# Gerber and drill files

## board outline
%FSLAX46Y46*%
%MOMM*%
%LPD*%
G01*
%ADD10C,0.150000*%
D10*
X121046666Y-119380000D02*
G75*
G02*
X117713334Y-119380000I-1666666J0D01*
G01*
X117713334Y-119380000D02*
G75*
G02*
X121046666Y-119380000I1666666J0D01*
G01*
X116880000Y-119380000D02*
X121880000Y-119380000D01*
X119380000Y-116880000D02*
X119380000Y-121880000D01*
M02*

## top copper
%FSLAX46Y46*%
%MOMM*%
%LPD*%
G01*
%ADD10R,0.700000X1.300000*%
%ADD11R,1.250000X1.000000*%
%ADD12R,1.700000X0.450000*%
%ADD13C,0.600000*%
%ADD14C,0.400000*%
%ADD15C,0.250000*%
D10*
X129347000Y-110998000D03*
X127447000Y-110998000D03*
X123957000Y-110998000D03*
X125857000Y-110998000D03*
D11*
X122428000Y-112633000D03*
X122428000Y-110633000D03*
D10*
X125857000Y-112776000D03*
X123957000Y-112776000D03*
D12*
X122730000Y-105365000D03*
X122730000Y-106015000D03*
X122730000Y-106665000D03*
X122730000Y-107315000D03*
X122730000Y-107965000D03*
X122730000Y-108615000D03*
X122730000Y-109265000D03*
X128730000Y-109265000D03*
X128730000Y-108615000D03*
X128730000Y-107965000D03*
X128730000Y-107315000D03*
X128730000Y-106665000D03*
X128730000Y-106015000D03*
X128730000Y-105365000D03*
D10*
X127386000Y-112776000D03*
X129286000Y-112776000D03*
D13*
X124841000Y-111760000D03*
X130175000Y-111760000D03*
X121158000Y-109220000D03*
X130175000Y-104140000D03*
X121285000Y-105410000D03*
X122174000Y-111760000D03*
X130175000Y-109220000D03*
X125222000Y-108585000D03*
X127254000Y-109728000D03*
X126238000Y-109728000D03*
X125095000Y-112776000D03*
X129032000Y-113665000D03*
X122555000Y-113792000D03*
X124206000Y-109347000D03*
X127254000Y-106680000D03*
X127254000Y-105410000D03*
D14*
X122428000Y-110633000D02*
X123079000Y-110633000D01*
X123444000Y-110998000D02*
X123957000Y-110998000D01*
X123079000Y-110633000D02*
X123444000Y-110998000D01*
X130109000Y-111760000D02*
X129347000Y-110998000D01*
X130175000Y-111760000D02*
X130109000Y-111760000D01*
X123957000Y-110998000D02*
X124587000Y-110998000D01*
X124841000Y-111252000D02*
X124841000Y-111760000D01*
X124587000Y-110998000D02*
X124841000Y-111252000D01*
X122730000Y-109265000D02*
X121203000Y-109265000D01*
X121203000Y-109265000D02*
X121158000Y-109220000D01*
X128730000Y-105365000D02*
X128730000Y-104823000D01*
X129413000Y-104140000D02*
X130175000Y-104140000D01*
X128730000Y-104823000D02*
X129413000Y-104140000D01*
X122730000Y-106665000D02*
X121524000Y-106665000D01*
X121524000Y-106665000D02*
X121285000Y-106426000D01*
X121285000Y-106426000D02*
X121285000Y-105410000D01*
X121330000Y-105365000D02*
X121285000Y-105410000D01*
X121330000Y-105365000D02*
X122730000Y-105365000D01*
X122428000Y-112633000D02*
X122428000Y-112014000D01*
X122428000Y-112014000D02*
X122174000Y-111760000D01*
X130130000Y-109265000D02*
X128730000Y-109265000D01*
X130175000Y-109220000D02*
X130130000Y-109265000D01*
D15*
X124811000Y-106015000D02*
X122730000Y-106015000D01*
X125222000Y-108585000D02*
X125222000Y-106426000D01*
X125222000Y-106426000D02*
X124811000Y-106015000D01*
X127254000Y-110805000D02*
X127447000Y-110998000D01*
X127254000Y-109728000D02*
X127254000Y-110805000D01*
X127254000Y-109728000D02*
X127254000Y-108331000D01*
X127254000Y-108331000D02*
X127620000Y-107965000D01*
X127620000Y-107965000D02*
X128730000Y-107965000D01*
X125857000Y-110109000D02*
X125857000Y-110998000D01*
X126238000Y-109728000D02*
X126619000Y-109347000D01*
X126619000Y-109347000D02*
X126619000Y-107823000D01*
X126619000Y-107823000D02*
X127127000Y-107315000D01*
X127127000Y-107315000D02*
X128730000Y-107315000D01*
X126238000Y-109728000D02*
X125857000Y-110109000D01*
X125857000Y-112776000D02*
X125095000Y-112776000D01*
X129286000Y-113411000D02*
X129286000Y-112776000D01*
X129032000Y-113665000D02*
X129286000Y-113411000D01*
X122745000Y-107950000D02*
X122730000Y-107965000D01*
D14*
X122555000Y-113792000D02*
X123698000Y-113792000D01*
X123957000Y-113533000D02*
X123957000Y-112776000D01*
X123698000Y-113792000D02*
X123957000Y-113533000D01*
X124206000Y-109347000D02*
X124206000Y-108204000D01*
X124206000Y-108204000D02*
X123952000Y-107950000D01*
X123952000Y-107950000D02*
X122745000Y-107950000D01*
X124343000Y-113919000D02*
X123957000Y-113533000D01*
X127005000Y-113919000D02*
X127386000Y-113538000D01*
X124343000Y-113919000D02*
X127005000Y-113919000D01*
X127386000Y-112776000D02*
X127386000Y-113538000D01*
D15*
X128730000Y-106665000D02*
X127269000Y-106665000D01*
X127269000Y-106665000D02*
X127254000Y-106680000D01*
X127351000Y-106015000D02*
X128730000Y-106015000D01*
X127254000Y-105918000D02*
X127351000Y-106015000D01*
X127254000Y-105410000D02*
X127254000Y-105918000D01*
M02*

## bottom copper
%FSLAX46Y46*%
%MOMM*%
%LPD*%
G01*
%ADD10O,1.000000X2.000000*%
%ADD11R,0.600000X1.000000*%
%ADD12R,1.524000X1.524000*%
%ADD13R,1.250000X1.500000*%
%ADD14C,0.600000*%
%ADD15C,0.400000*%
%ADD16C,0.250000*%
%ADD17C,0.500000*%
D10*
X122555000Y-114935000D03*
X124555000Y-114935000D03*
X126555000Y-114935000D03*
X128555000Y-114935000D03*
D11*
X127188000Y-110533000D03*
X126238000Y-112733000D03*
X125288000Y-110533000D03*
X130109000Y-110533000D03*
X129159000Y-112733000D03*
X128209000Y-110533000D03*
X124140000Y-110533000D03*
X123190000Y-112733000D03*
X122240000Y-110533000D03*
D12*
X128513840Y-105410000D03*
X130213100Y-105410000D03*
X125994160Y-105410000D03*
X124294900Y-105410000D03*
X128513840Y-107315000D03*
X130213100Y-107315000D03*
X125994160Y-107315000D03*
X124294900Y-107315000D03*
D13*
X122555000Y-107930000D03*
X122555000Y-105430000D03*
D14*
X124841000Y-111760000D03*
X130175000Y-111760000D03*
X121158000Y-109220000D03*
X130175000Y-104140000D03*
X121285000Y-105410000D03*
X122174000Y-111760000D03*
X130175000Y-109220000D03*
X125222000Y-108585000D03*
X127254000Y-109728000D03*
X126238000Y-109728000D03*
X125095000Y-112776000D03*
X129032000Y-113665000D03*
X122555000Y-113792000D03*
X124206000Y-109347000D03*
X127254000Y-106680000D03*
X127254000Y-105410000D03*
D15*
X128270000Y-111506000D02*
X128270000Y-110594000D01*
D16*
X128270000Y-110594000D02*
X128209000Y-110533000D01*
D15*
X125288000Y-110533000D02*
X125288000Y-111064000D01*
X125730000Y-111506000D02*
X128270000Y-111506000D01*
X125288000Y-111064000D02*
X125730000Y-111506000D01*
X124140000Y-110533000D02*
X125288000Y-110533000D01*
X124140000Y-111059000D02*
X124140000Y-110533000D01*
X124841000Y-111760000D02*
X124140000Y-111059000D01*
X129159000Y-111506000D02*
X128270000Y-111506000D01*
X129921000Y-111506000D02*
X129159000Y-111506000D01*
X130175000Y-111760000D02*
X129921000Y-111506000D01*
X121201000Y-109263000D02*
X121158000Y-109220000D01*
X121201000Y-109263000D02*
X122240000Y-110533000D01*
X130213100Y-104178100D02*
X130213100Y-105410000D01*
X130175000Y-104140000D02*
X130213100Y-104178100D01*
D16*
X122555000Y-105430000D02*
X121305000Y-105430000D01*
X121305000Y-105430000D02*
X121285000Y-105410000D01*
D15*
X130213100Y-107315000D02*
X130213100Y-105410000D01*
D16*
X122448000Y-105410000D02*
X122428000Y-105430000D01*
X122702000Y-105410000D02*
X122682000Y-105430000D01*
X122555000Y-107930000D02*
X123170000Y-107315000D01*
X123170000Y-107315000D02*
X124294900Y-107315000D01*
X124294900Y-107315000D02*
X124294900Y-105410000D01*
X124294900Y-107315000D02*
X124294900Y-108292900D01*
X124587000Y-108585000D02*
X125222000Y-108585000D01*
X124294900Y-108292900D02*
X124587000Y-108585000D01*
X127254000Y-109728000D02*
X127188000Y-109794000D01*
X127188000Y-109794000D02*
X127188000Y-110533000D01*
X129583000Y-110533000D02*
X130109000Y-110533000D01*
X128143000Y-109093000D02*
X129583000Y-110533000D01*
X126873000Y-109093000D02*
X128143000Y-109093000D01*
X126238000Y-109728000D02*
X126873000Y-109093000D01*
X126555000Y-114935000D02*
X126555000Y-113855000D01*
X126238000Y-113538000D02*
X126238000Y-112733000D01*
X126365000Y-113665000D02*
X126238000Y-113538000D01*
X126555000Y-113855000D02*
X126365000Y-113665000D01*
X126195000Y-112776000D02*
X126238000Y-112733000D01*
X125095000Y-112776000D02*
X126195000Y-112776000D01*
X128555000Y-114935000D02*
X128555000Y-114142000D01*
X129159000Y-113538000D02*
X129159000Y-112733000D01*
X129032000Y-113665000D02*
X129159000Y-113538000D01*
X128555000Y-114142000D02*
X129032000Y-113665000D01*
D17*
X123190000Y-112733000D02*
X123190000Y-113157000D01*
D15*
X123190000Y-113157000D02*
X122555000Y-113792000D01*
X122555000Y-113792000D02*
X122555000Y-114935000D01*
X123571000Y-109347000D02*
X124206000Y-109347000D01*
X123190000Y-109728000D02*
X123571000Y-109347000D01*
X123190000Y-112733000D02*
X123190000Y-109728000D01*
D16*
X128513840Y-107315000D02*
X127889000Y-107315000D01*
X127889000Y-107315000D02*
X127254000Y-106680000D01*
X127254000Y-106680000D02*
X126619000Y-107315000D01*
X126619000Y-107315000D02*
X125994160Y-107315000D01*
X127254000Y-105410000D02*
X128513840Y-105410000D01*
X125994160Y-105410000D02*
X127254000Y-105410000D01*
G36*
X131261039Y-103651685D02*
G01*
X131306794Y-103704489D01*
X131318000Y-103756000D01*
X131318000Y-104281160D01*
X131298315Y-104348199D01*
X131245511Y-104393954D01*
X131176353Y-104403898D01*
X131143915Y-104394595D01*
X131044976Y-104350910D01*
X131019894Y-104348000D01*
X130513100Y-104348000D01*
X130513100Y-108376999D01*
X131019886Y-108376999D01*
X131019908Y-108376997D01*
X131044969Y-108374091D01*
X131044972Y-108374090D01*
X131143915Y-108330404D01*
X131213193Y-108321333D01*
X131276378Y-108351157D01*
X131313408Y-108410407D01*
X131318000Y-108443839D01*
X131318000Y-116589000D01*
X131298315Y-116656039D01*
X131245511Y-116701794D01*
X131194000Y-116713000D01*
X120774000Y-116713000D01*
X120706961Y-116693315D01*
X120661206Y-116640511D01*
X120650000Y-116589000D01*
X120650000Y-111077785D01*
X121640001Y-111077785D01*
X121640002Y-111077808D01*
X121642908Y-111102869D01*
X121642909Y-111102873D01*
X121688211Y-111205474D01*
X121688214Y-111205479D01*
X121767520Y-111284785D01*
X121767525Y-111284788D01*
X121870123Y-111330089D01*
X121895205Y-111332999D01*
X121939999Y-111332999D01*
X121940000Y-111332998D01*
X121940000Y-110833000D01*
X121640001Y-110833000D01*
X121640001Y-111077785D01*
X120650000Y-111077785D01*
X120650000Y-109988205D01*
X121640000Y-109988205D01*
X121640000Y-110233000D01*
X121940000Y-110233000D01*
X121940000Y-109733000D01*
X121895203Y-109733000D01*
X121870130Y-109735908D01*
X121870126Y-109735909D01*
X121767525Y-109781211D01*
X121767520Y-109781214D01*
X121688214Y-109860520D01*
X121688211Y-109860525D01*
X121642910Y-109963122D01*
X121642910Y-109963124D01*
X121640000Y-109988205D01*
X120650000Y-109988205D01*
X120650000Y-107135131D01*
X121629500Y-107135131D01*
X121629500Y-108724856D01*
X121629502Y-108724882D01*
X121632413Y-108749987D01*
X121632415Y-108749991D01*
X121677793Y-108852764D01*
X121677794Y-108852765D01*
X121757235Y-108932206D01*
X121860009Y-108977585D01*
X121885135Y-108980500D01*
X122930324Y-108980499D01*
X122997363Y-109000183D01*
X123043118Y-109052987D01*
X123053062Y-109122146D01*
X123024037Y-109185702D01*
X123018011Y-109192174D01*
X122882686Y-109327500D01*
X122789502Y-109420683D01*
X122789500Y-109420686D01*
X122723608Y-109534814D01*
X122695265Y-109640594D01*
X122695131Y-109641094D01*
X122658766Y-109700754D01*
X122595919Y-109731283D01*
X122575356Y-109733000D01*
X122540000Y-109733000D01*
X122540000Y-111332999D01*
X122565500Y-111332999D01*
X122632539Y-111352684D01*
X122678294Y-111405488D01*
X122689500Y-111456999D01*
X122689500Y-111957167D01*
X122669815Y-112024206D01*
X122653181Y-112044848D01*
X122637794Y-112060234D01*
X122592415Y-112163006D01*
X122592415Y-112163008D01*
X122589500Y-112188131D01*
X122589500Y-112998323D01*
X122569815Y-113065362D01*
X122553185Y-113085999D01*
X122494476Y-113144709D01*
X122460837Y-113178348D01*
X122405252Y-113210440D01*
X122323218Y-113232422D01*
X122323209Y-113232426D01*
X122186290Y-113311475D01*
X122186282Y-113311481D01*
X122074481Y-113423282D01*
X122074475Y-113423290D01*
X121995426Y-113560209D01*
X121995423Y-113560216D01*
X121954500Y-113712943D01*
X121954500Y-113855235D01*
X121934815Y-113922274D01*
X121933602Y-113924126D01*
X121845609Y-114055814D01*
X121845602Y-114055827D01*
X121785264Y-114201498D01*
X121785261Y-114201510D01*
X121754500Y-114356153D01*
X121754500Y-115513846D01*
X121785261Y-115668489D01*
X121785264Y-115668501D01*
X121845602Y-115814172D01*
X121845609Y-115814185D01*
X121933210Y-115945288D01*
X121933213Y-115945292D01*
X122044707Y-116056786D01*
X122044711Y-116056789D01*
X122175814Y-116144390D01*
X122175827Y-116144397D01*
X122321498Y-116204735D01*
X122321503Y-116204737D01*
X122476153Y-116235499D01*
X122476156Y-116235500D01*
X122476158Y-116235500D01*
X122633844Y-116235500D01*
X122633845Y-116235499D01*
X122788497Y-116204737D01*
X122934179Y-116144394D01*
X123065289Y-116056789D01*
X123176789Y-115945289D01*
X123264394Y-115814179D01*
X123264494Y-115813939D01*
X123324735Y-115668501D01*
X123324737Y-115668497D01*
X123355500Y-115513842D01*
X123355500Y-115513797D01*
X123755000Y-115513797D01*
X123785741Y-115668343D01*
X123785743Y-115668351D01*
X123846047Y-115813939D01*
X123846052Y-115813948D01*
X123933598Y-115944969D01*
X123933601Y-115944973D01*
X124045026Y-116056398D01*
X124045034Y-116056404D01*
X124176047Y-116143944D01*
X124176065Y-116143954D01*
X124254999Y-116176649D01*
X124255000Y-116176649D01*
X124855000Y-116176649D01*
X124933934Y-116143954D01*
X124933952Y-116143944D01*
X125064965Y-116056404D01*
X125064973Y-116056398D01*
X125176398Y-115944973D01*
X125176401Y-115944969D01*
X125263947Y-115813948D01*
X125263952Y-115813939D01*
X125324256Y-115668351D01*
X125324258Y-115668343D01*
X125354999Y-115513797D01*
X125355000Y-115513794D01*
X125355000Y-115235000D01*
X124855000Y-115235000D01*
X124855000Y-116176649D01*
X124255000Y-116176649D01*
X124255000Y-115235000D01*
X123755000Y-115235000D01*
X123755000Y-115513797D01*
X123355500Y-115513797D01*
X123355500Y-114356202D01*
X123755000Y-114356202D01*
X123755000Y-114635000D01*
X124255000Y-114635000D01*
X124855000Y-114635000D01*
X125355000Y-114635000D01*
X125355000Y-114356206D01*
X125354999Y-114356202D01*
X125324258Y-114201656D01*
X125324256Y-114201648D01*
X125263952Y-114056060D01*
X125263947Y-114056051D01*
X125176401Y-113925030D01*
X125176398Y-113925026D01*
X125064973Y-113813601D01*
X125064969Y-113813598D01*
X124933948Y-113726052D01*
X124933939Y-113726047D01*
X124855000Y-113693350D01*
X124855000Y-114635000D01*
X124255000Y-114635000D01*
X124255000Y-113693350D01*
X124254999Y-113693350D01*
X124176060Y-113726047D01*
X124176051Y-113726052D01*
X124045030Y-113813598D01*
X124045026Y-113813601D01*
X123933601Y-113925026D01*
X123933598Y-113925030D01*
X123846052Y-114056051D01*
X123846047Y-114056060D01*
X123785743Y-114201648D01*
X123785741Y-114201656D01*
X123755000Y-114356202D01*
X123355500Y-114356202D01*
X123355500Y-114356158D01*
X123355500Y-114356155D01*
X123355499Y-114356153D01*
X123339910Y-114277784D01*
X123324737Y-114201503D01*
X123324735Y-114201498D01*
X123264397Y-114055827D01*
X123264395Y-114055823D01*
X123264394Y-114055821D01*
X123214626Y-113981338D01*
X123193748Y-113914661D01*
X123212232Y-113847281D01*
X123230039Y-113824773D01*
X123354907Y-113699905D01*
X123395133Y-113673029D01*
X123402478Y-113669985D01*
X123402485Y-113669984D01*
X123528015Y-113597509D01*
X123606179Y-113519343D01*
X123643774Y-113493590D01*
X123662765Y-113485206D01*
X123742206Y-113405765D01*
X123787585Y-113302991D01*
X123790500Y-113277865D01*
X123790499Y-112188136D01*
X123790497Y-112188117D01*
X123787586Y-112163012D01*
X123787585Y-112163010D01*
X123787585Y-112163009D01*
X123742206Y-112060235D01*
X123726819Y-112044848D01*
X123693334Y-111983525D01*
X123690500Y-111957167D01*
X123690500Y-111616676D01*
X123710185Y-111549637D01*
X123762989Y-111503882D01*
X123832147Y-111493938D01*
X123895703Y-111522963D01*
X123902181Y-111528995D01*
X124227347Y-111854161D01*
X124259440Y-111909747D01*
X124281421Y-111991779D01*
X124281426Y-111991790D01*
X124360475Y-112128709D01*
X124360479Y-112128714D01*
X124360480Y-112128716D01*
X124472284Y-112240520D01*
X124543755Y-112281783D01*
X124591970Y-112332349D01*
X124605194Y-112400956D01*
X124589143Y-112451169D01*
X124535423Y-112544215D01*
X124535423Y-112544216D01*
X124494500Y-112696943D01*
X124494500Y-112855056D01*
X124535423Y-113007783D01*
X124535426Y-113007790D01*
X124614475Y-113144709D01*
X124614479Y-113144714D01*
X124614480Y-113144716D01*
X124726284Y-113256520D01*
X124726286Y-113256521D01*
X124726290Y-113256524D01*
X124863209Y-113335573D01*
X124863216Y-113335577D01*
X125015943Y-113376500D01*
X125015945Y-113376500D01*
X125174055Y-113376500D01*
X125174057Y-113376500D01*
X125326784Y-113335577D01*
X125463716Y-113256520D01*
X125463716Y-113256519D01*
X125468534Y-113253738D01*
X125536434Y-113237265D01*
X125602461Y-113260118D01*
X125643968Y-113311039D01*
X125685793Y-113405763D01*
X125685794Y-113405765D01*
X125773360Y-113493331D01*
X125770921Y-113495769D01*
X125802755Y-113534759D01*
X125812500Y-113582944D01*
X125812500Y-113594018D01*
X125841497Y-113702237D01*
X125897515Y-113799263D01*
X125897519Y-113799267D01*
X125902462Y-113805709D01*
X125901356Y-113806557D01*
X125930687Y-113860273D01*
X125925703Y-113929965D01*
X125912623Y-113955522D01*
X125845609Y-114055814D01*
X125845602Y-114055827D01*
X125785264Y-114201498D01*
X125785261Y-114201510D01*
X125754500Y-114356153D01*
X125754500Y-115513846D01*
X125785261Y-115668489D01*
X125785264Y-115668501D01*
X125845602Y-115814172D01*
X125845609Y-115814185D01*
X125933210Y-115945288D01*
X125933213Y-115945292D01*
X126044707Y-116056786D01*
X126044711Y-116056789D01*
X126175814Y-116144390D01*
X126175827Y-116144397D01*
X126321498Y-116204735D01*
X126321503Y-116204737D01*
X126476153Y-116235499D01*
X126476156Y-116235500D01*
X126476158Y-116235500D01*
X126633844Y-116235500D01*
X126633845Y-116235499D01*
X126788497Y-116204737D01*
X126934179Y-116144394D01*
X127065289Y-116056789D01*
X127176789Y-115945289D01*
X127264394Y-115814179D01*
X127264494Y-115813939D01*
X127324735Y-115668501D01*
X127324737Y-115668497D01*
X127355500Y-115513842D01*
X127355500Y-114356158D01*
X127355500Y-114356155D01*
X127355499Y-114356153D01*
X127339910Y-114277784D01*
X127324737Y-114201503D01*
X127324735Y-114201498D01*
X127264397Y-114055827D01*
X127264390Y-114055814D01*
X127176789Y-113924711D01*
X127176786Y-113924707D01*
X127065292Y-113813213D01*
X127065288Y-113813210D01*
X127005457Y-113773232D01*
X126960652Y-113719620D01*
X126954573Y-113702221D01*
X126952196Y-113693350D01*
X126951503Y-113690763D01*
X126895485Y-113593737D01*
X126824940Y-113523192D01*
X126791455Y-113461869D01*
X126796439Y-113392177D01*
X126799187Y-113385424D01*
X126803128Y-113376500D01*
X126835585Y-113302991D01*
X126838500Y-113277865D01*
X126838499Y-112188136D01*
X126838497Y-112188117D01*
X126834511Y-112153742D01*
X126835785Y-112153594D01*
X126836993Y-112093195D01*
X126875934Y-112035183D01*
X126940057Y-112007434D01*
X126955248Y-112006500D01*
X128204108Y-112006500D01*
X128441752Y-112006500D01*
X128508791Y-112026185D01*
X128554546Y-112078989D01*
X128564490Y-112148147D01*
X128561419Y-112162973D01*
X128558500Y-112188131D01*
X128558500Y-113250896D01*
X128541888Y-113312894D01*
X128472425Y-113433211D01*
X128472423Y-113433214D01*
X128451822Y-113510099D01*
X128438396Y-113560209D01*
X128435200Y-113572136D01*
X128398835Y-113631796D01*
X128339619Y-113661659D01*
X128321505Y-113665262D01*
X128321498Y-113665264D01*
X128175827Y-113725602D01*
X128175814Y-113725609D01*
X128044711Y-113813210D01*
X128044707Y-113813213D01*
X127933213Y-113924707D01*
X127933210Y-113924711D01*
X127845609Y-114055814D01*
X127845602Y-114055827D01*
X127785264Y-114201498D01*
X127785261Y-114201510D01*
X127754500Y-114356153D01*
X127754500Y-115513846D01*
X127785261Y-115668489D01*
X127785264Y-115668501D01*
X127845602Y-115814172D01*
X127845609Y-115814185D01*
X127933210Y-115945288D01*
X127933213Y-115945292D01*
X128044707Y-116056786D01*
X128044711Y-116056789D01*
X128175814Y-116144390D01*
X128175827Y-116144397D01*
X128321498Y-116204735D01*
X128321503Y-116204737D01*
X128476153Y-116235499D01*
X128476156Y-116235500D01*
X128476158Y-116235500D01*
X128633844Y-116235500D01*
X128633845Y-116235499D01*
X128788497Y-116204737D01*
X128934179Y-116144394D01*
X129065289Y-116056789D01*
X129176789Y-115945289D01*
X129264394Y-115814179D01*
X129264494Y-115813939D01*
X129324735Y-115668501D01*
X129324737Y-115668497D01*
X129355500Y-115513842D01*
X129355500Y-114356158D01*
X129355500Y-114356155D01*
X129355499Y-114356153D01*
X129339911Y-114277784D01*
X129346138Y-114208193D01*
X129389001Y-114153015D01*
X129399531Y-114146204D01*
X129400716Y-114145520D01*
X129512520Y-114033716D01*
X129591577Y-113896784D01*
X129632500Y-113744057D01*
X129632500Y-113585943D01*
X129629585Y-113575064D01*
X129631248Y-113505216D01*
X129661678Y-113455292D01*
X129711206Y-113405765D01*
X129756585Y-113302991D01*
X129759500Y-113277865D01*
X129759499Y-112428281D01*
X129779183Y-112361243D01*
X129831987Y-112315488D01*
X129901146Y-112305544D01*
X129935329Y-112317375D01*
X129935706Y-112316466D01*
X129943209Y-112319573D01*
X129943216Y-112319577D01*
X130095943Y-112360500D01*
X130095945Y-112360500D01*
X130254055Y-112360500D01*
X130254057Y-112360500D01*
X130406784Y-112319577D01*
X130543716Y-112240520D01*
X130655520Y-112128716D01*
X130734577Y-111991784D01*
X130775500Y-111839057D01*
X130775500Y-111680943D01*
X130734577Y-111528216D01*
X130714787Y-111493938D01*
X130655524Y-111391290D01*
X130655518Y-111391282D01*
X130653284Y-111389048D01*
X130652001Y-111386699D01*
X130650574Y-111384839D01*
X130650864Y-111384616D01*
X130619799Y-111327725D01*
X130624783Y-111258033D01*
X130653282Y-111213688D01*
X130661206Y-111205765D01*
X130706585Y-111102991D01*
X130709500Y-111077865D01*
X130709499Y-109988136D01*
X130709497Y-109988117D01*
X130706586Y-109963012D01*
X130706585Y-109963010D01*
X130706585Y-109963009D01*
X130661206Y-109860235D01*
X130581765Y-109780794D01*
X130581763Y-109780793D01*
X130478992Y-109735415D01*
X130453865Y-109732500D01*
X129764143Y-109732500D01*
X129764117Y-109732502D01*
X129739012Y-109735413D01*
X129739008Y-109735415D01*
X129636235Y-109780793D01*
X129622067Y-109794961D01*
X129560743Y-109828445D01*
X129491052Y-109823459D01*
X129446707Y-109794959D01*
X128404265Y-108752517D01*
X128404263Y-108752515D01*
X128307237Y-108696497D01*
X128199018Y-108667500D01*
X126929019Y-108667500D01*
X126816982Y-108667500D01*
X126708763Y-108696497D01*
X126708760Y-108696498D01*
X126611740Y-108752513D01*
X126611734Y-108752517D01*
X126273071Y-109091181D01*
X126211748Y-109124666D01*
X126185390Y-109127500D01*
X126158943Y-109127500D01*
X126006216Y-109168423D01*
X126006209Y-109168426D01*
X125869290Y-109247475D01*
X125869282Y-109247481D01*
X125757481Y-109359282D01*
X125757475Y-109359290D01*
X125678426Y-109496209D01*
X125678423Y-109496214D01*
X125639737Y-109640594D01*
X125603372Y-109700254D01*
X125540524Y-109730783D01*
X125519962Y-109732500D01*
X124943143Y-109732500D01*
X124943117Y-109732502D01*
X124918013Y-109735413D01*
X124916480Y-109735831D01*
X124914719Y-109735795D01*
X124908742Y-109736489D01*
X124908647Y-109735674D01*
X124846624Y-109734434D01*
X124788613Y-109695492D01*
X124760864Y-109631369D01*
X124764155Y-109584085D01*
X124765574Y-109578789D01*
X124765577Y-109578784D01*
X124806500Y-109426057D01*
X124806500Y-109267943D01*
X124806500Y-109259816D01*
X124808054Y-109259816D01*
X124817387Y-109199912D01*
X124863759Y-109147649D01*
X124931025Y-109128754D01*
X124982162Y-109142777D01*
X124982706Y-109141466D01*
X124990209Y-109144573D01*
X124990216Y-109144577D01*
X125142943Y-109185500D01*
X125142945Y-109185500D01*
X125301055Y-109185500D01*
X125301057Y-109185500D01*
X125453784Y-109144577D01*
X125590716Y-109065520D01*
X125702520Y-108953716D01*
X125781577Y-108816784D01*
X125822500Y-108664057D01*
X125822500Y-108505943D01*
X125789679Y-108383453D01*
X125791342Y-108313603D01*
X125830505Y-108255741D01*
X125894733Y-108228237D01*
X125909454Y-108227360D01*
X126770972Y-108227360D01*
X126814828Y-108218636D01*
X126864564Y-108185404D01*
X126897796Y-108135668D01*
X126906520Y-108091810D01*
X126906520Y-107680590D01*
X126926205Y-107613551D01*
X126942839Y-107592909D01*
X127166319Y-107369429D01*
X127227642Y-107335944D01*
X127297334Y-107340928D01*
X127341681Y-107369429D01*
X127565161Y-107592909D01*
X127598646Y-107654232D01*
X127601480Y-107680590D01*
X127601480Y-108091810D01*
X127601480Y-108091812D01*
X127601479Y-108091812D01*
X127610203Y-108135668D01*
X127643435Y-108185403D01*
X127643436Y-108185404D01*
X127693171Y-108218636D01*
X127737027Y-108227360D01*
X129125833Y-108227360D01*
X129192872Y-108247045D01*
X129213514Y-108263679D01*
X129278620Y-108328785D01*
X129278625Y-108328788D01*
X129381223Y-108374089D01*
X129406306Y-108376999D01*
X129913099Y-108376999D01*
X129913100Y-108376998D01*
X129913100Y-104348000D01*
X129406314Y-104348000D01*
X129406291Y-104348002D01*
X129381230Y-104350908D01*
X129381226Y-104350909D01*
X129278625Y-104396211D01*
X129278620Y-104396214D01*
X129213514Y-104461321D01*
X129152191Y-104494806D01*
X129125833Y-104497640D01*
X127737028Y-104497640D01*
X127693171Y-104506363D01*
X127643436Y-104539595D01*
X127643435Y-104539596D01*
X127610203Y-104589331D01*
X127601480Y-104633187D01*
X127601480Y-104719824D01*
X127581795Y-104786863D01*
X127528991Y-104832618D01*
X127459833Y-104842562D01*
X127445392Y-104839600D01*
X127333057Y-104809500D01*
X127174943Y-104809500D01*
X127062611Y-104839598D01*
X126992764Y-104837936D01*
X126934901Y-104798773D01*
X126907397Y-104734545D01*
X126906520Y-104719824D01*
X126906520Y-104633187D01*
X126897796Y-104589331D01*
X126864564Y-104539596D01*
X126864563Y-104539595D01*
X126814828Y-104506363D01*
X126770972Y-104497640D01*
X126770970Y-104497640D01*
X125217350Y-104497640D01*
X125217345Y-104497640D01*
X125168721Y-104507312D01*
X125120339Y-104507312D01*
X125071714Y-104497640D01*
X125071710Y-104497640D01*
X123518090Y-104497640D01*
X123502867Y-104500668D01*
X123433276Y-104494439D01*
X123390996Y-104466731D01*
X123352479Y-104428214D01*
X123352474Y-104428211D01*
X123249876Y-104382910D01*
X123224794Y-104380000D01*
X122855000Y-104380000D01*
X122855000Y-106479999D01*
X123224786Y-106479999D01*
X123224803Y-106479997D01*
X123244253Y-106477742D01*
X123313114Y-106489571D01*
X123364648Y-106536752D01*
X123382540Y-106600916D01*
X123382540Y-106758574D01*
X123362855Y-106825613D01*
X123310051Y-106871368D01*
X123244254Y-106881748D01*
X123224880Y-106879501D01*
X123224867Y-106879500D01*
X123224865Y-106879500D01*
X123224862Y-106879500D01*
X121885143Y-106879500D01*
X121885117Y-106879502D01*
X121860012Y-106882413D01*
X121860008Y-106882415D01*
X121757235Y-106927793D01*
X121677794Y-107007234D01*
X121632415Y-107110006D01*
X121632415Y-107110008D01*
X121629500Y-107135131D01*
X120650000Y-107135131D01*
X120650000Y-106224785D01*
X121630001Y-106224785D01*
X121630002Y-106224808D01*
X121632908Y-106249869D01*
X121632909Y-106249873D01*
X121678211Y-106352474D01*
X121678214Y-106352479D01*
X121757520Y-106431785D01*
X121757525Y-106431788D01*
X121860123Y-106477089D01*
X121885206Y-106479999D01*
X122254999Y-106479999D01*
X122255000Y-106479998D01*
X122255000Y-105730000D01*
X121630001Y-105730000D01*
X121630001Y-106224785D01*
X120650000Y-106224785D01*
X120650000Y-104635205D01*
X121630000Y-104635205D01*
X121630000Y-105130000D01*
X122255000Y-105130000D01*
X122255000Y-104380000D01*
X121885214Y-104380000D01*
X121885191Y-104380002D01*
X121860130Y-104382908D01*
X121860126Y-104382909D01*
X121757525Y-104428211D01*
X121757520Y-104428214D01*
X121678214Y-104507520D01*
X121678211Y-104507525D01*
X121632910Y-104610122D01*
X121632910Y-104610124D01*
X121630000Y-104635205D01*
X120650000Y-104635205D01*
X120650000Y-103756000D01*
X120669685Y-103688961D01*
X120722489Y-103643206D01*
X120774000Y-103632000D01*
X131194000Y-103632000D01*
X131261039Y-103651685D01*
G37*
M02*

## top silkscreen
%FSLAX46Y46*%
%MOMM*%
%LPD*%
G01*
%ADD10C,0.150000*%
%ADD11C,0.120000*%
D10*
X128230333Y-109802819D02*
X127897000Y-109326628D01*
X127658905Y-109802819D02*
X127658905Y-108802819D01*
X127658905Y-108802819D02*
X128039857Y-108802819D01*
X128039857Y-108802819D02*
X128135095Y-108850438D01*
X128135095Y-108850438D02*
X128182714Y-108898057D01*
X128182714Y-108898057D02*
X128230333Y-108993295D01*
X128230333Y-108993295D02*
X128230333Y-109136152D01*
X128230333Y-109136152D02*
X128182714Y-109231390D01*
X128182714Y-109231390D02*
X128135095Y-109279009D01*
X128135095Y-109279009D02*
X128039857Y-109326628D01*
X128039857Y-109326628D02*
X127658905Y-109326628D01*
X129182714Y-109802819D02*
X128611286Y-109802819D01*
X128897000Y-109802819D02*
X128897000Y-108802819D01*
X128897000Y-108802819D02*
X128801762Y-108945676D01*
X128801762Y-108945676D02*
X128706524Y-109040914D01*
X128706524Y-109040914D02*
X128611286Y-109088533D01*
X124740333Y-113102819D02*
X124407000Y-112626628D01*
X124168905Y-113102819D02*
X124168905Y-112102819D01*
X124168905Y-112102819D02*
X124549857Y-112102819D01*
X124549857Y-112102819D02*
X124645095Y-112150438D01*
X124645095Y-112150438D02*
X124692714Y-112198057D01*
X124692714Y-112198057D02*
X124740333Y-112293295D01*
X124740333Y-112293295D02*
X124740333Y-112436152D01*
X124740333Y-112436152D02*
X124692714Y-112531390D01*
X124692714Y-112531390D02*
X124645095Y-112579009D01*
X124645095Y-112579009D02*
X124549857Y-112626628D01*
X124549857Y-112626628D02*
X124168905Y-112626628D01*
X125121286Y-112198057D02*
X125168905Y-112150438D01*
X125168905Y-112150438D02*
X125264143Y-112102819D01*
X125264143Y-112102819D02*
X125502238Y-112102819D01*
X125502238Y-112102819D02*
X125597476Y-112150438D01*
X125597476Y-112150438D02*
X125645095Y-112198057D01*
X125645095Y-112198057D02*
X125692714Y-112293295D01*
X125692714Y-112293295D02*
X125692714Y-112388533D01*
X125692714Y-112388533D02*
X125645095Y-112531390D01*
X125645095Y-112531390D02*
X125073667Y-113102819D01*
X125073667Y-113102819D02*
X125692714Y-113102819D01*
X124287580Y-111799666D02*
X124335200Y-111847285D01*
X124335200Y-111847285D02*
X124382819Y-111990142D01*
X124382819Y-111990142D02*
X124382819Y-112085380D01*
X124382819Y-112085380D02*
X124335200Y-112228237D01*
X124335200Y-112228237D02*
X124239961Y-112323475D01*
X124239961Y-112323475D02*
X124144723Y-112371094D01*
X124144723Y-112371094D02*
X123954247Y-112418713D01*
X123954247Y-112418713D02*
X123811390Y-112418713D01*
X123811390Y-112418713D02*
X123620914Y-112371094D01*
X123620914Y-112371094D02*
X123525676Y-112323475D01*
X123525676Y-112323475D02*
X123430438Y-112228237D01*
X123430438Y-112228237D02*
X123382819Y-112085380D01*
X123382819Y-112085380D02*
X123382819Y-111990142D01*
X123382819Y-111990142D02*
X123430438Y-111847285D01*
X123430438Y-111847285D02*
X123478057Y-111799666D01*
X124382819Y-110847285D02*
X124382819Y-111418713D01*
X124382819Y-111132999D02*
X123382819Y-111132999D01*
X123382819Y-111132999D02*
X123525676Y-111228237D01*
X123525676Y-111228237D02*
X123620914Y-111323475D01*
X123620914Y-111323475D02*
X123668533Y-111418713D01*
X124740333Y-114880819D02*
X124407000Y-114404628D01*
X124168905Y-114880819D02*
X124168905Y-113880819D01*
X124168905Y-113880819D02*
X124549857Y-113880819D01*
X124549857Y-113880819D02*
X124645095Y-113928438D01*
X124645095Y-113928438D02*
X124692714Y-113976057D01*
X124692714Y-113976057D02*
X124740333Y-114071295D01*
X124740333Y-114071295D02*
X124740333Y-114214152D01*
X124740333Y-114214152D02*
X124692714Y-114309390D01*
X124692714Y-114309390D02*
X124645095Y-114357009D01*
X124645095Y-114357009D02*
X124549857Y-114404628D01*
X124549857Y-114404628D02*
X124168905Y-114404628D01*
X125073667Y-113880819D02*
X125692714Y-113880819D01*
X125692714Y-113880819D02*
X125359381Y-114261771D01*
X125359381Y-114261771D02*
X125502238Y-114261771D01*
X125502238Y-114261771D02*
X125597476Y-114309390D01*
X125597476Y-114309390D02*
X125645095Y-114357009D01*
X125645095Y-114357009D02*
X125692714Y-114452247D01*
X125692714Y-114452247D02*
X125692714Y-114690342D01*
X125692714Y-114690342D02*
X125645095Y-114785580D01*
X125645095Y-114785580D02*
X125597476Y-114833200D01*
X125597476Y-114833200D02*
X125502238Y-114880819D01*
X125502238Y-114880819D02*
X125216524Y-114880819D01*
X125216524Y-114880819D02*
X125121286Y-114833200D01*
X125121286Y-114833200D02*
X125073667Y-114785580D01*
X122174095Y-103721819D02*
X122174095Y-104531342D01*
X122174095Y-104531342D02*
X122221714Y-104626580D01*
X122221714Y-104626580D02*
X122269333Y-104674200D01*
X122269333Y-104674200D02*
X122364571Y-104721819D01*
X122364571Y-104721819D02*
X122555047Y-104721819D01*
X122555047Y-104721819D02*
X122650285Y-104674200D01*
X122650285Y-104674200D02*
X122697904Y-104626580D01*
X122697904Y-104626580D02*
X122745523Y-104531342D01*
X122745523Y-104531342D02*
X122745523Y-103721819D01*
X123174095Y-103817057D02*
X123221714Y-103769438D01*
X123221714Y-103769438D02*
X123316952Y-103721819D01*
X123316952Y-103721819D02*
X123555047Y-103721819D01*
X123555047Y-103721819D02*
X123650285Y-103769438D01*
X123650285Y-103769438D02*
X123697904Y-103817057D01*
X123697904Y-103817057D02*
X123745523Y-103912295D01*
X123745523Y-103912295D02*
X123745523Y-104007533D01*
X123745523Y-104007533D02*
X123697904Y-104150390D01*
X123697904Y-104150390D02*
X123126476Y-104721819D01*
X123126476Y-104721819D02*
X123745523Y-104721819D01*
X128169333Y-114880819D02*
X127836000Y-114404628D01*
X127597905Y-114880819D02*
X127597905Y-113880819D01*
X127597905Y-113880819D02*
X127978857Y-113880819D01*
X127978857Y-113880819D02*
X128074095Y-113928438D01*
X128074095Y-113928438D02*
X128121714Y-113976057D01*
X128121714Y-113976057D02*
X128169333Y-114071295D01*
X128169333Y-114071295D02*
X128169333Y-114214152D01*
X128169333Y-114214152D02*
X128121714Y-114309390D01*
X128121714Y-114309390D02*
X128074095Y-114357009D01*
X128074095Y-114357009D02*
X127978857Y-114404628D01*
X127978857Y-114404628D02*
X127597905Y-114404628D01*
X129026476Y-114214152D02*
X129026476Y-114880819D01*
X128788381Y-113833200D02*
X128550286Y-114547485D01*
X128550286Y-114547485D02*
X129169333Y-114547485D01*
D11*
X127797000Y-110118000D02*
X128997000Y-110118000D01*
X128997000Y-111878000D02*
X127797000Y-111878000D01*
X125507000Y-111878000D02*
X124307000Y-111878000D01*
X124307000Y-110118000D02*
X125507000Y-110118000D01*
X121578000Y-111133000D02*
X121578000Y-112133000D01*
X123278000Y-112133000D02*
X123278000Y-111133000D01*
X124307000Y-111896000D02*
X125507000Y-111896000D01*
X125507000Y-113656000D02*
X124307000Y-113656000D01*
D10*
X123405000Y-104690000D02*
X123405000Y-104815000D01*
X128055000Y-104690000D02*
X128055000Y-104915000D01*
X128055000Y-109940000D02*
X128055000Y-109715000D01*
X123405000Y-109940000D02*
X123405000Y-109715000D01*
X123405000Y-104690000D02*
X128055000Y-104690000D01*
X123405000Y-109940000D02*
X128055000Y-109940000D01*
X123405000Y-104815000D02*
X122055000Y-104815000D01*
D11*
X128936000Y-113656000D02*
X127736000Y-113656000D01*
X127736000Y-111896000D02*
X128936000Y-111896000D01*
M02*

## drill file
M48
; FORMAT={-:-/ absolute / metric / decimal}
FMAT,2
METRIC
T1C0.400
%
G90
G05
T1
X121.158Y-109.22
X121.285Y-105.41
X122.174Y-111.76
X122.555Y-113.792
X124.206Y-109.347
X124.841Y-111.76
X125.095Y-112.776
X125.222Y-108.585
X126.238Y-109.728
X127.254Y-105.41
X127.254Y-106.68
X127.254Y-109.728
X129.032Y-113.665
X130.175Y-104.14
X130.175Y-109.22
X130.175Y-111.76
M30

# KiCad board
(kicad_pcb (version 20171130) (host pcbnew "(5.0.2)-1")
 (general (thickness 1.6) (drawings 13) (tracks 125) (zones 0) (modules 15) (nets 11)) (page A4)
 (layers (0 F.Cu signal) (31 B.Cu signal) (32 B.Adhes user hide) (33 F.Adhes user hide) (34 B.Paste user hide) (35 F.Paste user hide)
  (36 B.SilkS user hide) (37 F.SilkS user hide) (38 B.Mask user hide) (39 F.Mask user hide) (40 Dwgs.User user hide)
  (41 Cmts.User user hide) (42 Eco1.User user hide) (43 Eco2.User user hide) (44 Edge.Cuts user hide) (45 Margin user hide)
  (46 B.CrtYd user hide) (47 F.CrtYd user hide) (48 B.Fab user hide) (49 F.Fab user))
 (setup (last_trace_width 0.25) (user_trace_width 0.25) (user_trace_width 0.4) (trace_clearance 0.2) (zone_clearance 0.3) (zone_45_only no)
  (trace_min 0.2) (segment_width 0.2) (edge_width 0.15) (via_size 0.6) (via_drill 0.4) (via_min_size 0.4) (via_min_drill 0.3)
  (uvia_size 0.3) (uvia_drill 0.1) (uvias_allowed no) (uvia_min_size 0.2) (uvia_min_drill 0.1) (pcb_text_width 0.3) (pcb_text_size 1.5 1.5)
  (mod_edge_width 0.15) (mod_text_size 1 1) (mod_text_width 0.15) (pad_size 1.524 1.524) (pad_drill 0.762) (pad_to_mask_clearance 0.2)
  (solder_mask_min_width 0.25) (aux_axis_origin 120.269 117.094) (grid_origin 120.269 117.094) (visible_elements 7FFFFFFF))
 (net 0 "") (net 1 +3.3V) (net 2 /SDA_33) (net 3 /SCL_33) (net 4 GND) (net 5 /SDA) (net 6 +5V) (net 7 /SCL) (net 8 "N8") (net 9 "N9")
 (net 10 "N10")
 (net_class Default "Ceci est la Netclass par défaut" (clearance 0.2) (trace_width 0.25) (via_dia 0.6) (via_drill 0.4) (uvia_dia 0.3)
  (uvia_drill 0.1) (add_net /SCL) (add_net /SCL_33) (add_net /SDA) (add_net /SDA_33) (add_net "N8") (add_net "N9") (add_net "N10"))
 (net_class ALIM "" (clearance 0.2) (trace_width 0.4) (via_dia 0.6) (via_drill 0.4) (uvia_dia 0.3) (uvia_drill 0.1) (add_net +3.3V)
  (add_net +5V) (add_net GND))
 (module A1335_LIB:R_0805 (layer F.Cu) (at 128.397 110.998)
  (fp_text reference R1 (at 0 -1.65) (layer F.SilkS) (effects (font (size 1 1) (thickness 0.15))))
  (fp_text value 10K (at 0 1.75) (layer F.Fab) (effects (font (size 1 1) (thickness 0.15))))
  (fp_line (start -0.6 -0.88) (end 0.6 -0.88) (layer F.SilkS) (width 0.12))
  (fp_line (start 0.6 0.88) (end -0.6 0.88) (layer F.SilkS) (width 0.12))
  (pad 2 smd rect (at 0.95 0) (size 0.7 1.3) (layers F.Cu F.Paste F.Mask) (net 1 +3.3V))
  (pad 1 smd rect (at -0.95 0) (size 0.7 1.3) (layers F.Cu F.Paste F.Mask) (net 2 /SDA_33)))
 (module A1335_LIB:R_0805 (layer F.Cu) (at 124.907 110.998 180)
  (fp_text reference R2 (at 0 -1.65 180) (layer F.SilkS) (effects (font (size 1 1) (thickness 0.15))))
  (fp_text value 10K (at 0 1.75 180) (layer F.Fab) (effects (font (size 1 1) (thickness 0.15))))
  (fp_line (start -0.6 -0.88) (end 0.6 -0.88) (layer F.SilkS) (width 0.12))
  (fp_line (start 0.6 0.88) (end -0.6 0.88) (layer F.SilkS) (width 0.12))
  (pad 2 smd rect (at 0.95 0 180) (size 0.7 1.3) (layers F.Cu F.Paste F.Mask) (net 1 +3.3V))
  (pad 1 smd rect (at -0.95 0 180) (size 0.7 1.3) (layers F.Cu F.Paste F.Mask) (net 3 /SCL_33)))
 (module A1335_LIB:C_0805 (layer F.Cu) (at 122.428 111.633 270)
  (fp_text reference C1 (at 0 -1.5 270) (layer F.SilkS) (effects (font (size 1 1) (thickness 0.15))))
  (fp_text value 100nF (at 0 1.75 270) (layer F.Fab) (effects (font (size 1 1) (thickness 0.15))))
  (fp_line (start -0.5 0.85) (end 0.5 0.85) (layer F.SilkS) (width 0.12))
  (fp_line (start 0.5 -0.85) (end -0.5 -0.85) (layer F.SilkS) (width 0.12))
  (pad 2 smd rect (at 1 0 270) (size 1 1.25) (layers F.Cu F.Paste F.Mask) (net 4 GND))
  (pad 1 smd rect (at -1 0 270) (size 1 1.25) (layers F.Cu F.Paste F.Mask) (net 1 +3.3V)))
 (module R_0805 (layer F.Cu) (at 124.907 112.776 180)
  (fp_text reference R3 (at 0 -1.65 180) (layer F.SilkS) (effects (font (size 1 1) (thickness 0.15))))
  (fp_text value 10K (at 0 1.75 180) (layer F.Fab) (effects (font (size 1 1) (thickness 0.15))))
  (fp_line (start 0.6 0.88) (end -0.6 0.88) (layer F.SilkS) (width 0.12))
  (fp_line (start -0.6 -0.88) (end 0.6 -0.88) (layer F.SilkS) (width 0.12))
  (pad 1 smd rect (at -0.95 0 180) (size 0.7 1.3) (layers F.Cu F.Paste F.Mask) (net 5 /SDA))
  (pad 2 smd rect (at 0.95 0 180) (size 0.7 1.3) (layers F.Cu F.Paste F.Mask) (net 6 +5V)))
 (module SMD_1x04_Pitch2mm (layer B.Cu) (at 122.555 114.935 270)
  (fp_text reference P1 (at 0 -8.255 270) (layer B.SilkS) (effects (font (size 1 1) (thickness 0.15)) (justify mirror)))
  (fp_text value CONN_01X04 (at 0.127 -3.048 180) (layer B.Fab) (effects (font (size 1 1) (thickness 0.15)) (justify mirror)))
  (pad 1 smd oval (at 0 0 270) (size 2 1) (layers B.Cu B.Paste B.Mask) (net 6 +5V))
  (pad 2 smd oval (at 0 -2 270) (size 2 1) (layers B.Cu B.Paste B.Mask) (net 4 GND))
  (pad 3 smd oval (at 0 -4 270) (size 2 1) (layers B.Cu B.Paste B.Mask) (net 5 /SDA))
  (pad 4 smd oval (at 0 -6 270) (size 2 1) (layers B.Cu B.Paste B.Mask) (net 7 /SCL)))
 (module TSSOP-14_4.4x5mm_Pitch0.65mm (layer F.Cu) (at 125.73 107.315)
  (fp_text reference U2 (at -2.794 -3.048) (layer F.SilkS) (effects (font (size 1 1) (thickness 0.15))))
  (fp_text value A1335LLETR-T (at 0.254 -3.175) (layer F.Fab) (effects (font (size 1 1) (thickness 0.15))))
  (fp_line (start -2.325 -2.625) (end -2.325 -2.5) (layer F.SilkS) (width 0.15))
  (fp_line (start 2.325 -2.625) (end 2.325 -2.4) (layer F.SilkS) (width 0.15))
  (fp_line (start 2.325 2.625) (end 2.325 2.4) (layer F.SilkS) (width 0.15))
  (fp_line (start -2.325 2.625) (end -2.325 2.4) (layer F.SilkS) (width 0.15))
  (fp_line (start -2.325 -2.625) (end 2.325 -2.625) (layer F.SilkS) (width 0.15))
  (fp_line (start -2.325 2.625) (end 2.325 2.625) (layer F.SilkS) (width 0.15))
  (fp_line (start -2.325 -2.5) (end -3.675 -2.5) (layer F.SilkS) (width 0.15))
  (pad 1 smd rect (at -3 -1.95) (size 1.7 0.45) (layers F.Cu F.Paste F.Mask) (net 4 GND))
  (pad 2 smd rect (at -3 -1.3) (size 1.7 0.45) (layers F.Cu F.Paste F.Mask) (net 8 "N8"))
  (pad 3 smd rect (at -3 -0.65) (size 1.7 0.45) (layers F.Cu F.Paste F.Mask) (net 4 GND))
  (pad 4 smd rect (at -3 0) (size 1.7 0.45) (layers F.Cu F.Paste F.Mask))
  (pad 5 smd rect (at -3 0.65) (size 1.7 0.45) (layers F.Cu F.Paste F.Mask) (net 6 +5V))
  (pad 6 smd rect (at -3 1.3) (size 1.7 0.45) (layers F.Cu F.Paste F.Mask))
  (pad 7 smd rect (at -3 1.95) (size 1.7 0.45) (layers F.Cu F.Paste F.Mask) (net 4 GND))
  (pad 8 smd rect (at 3 1.95) (size 1.7 0.45) (layers F.Cu F.Paste F.Mask) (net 4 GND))
  (pad 9 smd rect (at 3 1.3) (size 1.7 0.45) (layers F.Cu F.Paste F.Mask))
  (pad 10 smd rect (at 3 0.65) (size 1.7 0.45) (layers F.Cu F.Paste F.Mask) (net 2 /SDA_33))
  (pad 11 smd rect (at 3 0) (size 1.7 0.45) (layers F.Cu F.Paste F.Mask) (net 3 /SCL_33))
  (pad 12 smd rect (at 3 -0.65) (size 1.7 0.45) (layers F.Cu F.Paste F.Mask) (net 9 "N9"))
  (pad 13 smd rect (at 3 -1.3) (size 1.7 0.45) (layers F.Cu F.Paste F.Mask) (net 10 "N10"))
  (pad 14 smd rect (at 3 -1.95) (size 1.7 0.45) (layers F.Cu F.Paste F.Mask) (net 4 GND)))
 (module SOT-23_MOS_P (layer B.Cu) (at 126.238 111.633)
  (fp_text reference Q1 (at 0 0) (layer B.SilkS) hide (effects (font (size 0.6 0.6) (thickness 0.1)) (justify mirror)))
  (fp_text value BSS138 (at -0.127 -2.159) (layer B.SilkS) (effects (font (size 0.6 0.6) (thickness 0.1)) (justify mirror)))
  (pad S smd rect (at 0.95 -1.1) (size 0.6 1) (layers B.Cu B.Mask) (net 2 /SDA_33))
  (pad D smd rect (at 0 1.1) (size 0.6 1) (layers B.Cu B.Mask) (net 5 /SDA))
  (pad G smd rect (at -0.95 -1.1) (size 0.6 1) (layers B.Cu B.Mask) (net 1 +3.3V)))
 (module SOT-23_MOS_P (layer B.Cu) (at 129.159 111.633)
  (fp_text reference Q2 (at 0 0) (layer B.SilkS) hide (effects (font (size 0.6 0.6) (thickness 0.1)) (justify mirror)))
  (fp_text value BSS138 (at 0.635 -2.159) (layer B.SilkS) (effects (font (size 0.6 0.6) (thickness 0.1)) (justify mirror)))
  (pad S smd rect (at 0.95 -1.1) (size 0.6 1) (layers B.Cu B.Mask) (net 3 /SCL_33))
  (pad D smd rect (at 0 1.1) (size 0.6 1) (layers B.Cu B.Mask) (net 7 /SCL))
  (pad G smd rect (at -0.95 -1.1) (size 0.6 1) (layers B.Cu B.Mask) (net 1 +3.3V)))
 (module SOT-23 (layer B.Cu) (at 123.19 111.633)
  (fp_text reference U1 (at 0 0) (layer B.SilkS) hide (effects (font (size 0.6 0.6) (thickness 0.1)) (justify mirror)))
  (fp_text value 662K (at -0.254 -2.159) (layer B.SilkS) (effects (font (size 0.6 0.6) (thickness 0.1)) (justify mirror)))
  (pad 2 smd rect (at 0.95 -1.1) (size 0.6 1) (layers B.Cu B.Mask) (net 1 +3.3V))
  (pad 3 smd rect (at 0 1.1) (size 0.6 1) (layers B.Cu B.Mask) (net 6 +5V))
  (pad 1 smd rect (at -0.95 -1.1) (size 0.6 1) (layers B.Cu B.Mask) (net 4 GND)))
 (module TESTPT (layer B.Cu) (at 129.413 105.41)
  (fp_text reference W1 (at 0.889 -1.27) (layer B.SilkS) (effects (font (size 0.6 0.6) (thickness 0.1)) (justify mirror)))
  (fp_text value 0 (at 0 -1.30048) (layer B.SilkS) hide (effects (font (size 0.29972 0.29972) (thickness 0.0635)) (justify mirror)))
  (pad 1 smd rect (at -0.89916 0) (size 1.524 1.524) (layers B.Cu B.Paste B.Mask) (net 10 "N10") (clearance 0.14986))
  (pad 2 smd rect (at 0.8001 0) (size 1.524 1.524) (layers B.Cu B.Paste B.Mask) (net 4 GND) (clearance 0.14986)))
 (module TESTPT (layer B.Cu) (at 125.095 105.41 180)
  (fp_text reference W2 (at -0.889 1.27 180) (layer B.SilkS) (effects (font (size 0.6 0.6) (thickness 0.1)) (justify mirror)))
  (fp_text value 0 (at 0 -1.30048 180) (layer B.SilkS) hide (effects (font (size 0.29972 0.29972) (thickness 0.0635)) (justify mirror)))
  (pad 1 smd rect (at -0.89916 0 180) (size 1.524 1.524) (layers B.Cu B.Paste B.Mask) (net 10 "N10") (clearance 0.14986))
  (pad 2 smd rect (at 0.8001 0 180) (size 1.524 1.524) (layers B.Cu B.Paste B.Mask) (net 8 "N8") (clearance 0.14986)))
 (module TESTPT (layer B.Cu) (at 129.413 107.315)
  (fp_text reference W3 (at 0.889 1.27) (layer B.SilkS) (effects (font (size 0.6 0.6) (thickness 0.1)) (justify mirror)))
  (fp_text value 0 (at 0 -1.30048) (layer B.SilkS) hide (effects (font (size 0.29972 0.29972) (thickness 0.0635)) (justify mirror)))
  (pad 1 smd rect (at -0.89916 0) (size 1.524 1.524) (layers B.Cu B.Paste B.Mask) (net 9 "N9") (clearance 0.14986))
  (pad 2 smd rect (at 0.8001 0) (size 1.524 1.524) (layers B.Cu B.Paste B.Mask) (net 4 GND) (clearance 0.14986)))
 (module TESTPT (layer B.Cu) (at 125.095 107.315 180)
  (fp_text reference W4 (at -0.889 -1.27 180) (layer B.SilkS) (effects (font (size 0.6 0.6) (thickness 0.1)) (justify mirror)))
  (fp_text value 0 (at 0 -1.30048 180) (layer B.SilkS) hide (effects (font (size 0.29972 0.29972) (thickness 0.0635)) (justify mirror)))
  (pad 1 smd rect (at -0.89916 0 180) (size 1.524 1.524) (layers B.Cu B.Paste B.Mask) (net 9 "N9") (clearance 0.14986))
  (pad 2 smd rect (at 0.8001 0 180) (size 1.524 1.524) (layers B.Cu B.Paste B.Mask) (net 8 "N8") (clearance 0.14986)))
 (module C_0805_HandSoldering (layer B.Cu) (at 122.555 106.68 90)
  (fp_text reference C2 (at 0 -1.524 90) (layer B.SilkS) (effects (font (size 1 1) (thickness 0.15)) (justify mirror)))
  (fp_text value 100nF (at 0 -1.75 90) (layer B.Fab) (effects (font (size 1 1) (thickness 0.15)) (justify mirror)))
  (pad 1 smd rect (at -1.25 0 90) (size 1.5 1.25) (layers B.Cu B.Paste B.Mask) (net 8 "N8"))
  (pad 2 smd rect (at 1.25 0 90) (size 1.5 1.25) (layers B.Cu B.Paste B.Mask) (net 4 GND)))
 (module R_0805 (layer F.Cu) (at 128.336 112.776 180)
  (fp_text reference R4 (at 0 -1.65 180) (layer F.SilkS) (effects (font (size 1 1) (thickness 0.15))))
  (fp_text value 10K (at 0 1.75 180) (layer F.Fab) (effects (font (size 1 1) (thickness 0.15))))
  (fp_line (start -0.6 -0.88) (end 0.6 -0.88) (layer F.SilkS) (width 0.12))
  (fp_line (start 0.6 0.88) (end -0.6 0.88) (layer F.SilkS) (width 0.12))
  (pad 2 smd rect (at 0.95 0 180) (size 0.7 1.3) (layers F.Cu F.Paste F.Mask) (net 6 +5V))
  (pad 1 smd rect (at -0.95 0 180) (size 0.7 1.3) (layers F.Cu F.Paste F.Mask) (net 7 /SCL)))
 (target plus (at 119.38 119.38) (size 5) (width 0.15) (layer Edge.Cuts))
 (segment (start 128.27 111.506) (end 128.27 110.594) (width 0.4) (layer B.Cu) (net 1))
 (segment (start 128.27 110.594) (end 128.209 110.533) (width 0.25) (layer B.Cu) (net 1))
 (segment (start 125.288 110.533) (end 125.288 111.064) (width 0.4) (layer B.Cu) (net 1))
 (segment (start 125.73 111.506) (end 128.27 111.506) (width 0.4) (layer B.Cu) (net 1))
 (segment (start 125.288 111.064) (end 125.73 111.506) (width 0.4) (layer B.Cu) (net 1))
 (segment (start 124.14 110.533) (end 125.288 110.533) (width 0.4) (layer B.Cu) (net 1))
 (segment (start 122.428 110.633) (end 123.079 110.633) (width 0.4) (layer F.Cu) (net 1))
 (segment (start 123.444 110.998) (end 123.957 110.998) (width 0.4) (layer F.Cu) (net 1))
 (segment (start 123.079 110.633) (end 123.444 110.998) (width 0.4) (layer F.Cu) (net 1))
 (segment (start 124.14 111.059) (end 124.14 110.533) (width 0.4) (layer B.Cu) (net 1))
 (via (at 124.841 111.76) (size 0.6) (drill 0.4) (layers F.Cu B.Cu) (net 1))
 (segment (start 124.841 111.76) (end 124.14 111.059) (width 0.4) (layer B.Cu) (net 1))
 (segment (start 129.159 111.506) (end 128.27 111.506) (width 0.4) (layer B.Cu) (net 1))
 (segment (start 129.921 111.506) (end 129.159 111.506) (width 0.4) (layer B.Cu) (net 1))
 (segment (start 130.175 111.76) (end 129.921 111.506) (width 0.4) (layer B.Cu) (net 1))
 (via (at 130.175 111.76) (size 0.6) (drill 0.4) (layers F.Cu B.Cu) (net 1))
 (segment (start 130.109 111.76) (end 129.347 110.998) (width 0.4) (layer F.Cu) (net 1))
 (segment (start 130.175 111.76) (end 130.109 111.76) (width 0.4) (layer F.Cu) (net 1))
 (segment (start 123.957 110.998) (end 124.587 110.998) (width 0.4) (layer F.Cu) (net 1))
 (segment (start 124.841 111.252) (end 124.841 111.76) (width 0.4) (layer F.Cu) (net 1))
 (segment (start 124.587 110.998) (end 124.841 111.252) (width 0.4) (layer F.Cu) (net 1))
 (segment (start 122.73 109.265) (end 121.203 109.265) (width 0.4) (layer F.Cu) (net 4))
 (segment (start 121.203 109.265) (end 121.158 109.22) (width 0.4) (layer F.Cu) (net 4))
 (segment (start 121.201 109.263) (end 121.158 109.22) (width 0.4) (layer B.Cu) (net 4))
 (segment (start 121.201 109.263) (end 122.24 110.533) (width 0.4) (layer B.Cu) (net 4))
 (via (at 121.158 109.22) (size 0.6) (drill 0.4) (layers F.Cu B.Cu) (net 4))
 (segment (start 128.73 105.365) (end 128.73 104.823) (width 0.4) (layer F.Cu) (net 4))
 (segment (start 130.2131 104.1781) (end 130.2131 105.41) (width 0.4) (layer B.Cu) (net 4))
 (segment (start 130.175 104.14) (end 130.2131 104.1781) (width 0.4) (layer B.Cu) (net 4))
 (via (at 130.175 104.14) (size 0.6) (drill 0.4) (layers F.Cu B.Cu) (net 4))
 (segment (start 129.413 104.14) (end 130.175 104.14) (width 0.4) (layer F.Cu) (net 4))
 (segment (start 128.73 104.823) (end 129.413 104.14) (width 0.4) (layer F.Cu) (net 4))
 (segment (start 122.73 106.665) (end 121.524 106.665) (width 0.4) (layer F.Cu) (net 4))
 (segment (start 121.524 106.665) (end 121.285 106.426) (width 0.4) (layer F.Cu) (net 4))
 (segment (start 121.285 106.426) (end 121.285 105.41) (width 0.4) (layer F.Cu) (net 4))
 (segment (start 122.555 105.43) (end 121.305 105.43) (width 0.25) (layer B.Cu) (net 4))
 (segment (start 121.33 105.365) (end 121.285 105.41) (width 0.4) (layer F.Cu) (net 4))
 (segment (start 121.33 105.365) (end 122.73 105.365) (width 0.4) (layer F.Cu) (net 4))
 (via (at 121.285 105.41) (size 0.6) (drill 0.4) (layers F.Cu B.Cu) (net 4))
 (segment (start 121.305 105.43) (end 121.285 105.41) (width 0.25) (layer B.Cu) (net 4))
 (segment (start 130.2131 107.315) (end 130.2131 105.41) (width 0.4) (layer B.Cu) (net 4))
 (segment (start 122.448 105.41) (end 122.428 105.43) (width 0.25) (layer B.Cu) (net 4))
 (segment (start 122.702 105.41) (end 122.682 105.43) (width 0.25) (layer B.Cu) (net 4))
 (segment (start 122.428 112.633) (end 122.428 112.014) (width 0.4) (layer F.Cu) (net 4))
 (via (at 122.174 111.76) (size 0.6) (drill 0.4) (layers F.Cu B.Cu) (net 4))
 (segment (start 122.428 112.014) (end 122.174 111.76) (width 0.4) (layer F.Cu) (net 4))
 (segment (start 130.13 109.265) (end 128.73 109.265) (width 0.4) (layer F.Cu) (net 4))
 (via (at 130.175 109.22) (size 0.6) (drill 0.4) (layers F.Cu B.Cu) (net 4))
 (segment (start 130.175 109.22) (end 130.13 109.265) (width 0.4) (layer F.Cu) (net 4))
 (segment (start 122.555 107.93) (end 123.17 107.315) (width 0.25) (layer B.Cu) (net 8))
 (segment (start 123.17 107.315) (end 124.2949 107.315) (width 0.25) (layer B.Cu) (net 8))
 (segment (start 124.2949 107.315) (end 124.2949 105.41) (width 0.25) (layer B.Cu) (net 8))
 (segment (start 124.811 106.015) (end 122.73 106.015) (width 0.25) (layer F.Cu) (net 8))
 (via (at 125.222 108.585) (size 0.6) (drill 0.4) (layers F.Cu B.Cu) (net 8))
 (segment (start 125.222 108.585) (end 125.222 106.426) (width 0.25) (layer F.Cu) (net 8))
 (segment (start 125.222 106.426) (end 124.811 106.015) (width 0.25) (layer F.Cu) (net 8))
 (segment (start 124.2949 107.315) (end 124.2949 108.2929) (width 0.25) (layer B.Cu) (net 8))
 (segment (start 124.587 108.585) (end 125.222 108.585) (width 0.25) (layer B.Cu) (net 8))
 (segment (start 124.2949 108.2929) (end 124.587 108.585) (width 0.25) (layer B.Cu) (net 8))
 (segment (start 127.254 110.805) (end 127.447 110.998) (width 0.25) (layer F.Cu) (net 2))
 (segment (start 127.254 109.728) (end 127.254 110.805) (width 0.25) (layer F.Cu) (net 2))
 (via (at 127.254 109.728) (size 0.6) (drill 0.4) (layers F.Cu B.Cu) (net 2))
 (segment (start 127.254 109.728) (end 127.188 109.794) (width 0.25) (layer B.Cu) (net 2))
 (segment (start 127.254 109.728) (end 127.254 108.331) (width 0.25) (layer F.Cu) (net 2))
 (segment (start 127.254 108.331) (end 127.62 107.965) (width 0.25) (layer F.Cu) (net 2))
 (segment (start 127.62 107.965) (end 128.73 107.965) (width 0.25) (layer F.Cu) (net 2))
 (segment (start 127.188 109.794) (end 127.188 110.533) (width 0.25) (layer B.Cu) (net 2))
 (segment (start 129.583 110.533) (end 130.109 110.533) (width 0.25) (layer B.Cu) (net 3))
 (segment (start 128.143 109.093) (end 129.583 110.533) (width 0.25) (layer B.Cu) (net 3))
 (segment (start 126.873 109.093) (end 128.143 109.093) (width 0.25) (layer B.Cu) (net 3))
 (segment (start 126.238 109.728) (end 126.873 109.093) (width 0.25) (layer B.Cu) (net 3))
 (segment (start 125.857 110.109) (end 125.857 110.998) (width 0.25) (layer F.Cu) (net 3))
 (via (at 126.238 109.728) (size 0.6) (drill 0.4) (layers F.Cu B.Cu) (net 3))
 (segment (start 126.238 109.728) (end 126.619 109.347) (width 0.25) (layer F.Cu) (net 3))
 (segment (start 126.619 109.347) (end 126.619 107.823) (width 0.25) (layer F.Cu) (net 3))
 (segment (start 126.619 107.823) (end 127.127 107.315) (width 0.25) (layer F.Cu) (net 3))
 (segment (start 127.127 107.315) (end 128.73 107.315) (width 0.25) (layer F.Cu) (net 3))
 (segment (start 126.238 109.728) (end 125.857 110.109) (width 0.25) (layer F.Cu) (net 3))
 (segment (start 126.555 114.935) (end 126.555 113.855) (width 0.25) (layer B.Cu) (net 5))
 (segment (start 126.238 113.538) (end 126.238 112.733) (width 0.25) (layer B.Cu) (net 5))
 (segment (start 126.365 113.665) (end 126.238 113.538) (width 0.25) (layer B.Cu) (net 5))
 (segment (start 126.555 113.855) (end 126.365 113.665) (width 0.25) (layer B.Cu) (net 5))
 (segment (start 125.857 112.776) (end 125.095 112.776) (width 0.25) (layer F.Cu) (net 5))
 (via (at 125.095 112.776) (size 0.6) (drill 0.4) (layers F.Cu B.Cu) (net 5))
 (segment (start 126.195 112.776) (end 126.238 112.733) (width 0.25) (layer B.Cu) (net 5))
 (segment (start 125.095 112.776) (end 126.195 112.776) (width 0.25) (layer B.Cu) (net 5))
 (segment (start 128.555 114.935) (end 128.555 114.142) (width 0.25) (layer B.Cu) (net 7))
 (segment (start 129.159 113.538) (end 129.159 112.733) (width 0.25) (layer B.Cu) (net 7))
 (via (at 129.032 113.665) (size 0.6) (drill 0.4) (layers F.Cu B.Cu) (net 7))
 (segment (start 129.032 113.665) (end 129.159 113.538) (width 0.25) (layer B.Cu) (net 7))
 (segment (start 128.555 114.142) (end 129.032 113.665) (width 0.25) (layer B.Cu) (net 7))
 (segment (start 129.286 113.411) (end 129.286 112.776) (width 0.25) (layer F.Cu) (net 7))
 (segment (start 129.032 113.665) (end 129.286 113.411) (width 0.25) (layer F.Cu) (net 7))
 (segment (start 122.745 107.95) (end 122.73 107.965) (width 0.25) (layer F.Cu) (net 6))
 (segment (start 123.19 112.733) (end 123.19 113.157) (width 0.5) (layer B.Cu) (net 6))
 (segment (start 123.19 113.157) (end 122.555 113.792) (width 0.4) (layer B.Cu) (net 6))
 (segment (start 122.555 113.792) (end 122.555 114.935) (width 0.4) (layer B.Cu) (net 6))
 (via (at 122.555 113.792) (size 0.6) (drill 0.4) (layers F.Cu B.Cu) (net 6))
 (segment (start 122.555 113.792) (end 123.698 113.792) (width 0.4) (layer F.Cu) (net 6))
 (segment (start 123.957 113.533) (end 123.957 112.776) (width 0.4) (layer F.Cu) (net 6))
 (segment (start 123.698 113.792) (end 123.957 113.533) (width 0.4) (layer F.Cu) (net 6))
 (segment (start 124.206 109.347) (end 124.206 108.204) (width 0.4) (layer F.Cu) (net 6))
 (segment (start 124.206 108.204) (end 123.952 107.95) (width 0.4) (layer F.Cu) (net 6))
 (via (at 124.206 109.347) (size 0.6) (drill 0.4) (layers F.Cu B.Cu) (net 6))
 (segment (start 123.952 107.95) (end 122.745 107.95) (width 0.4) (layer F.Cu) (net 6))
 (segment (start 123.571 109.347) (end 124.206 109.347) (width 0.4) (layer B.Cu) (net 6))
 (segment (start 123.19 109.728) (end 123.571 109.347) (width 0.4) (layer B.Cu) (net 6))
 (segment (start 123.19 112.733) (end 123.19 109.728) (width 0.4) (layer B.Cu) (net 6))
 (segment (start 124.343 113.919) (end 123.957 113.533) (width 0.4) (layer F.Cu) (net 6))
 (segment (start 127.005 113.919) (end 127.386 113.538) (width 0.4) (layer F.Cu) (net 6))
 (segment (start 124.343 113.919) (end 127.005 113.919) (width 0.4) (layer F.Cu) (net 6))
 (segment (start 127.386 112.776) (end 127.386 113.538) (width 0.4) (layer F.Cu) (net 6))
 (segment (start 128.51384 107.315) (end 127.889 107.315) (width 0.25) (layer B.Cu) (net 9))
 (segment (start 127.889 107.315) (end 127.254 106.68) (width 0.25) (layer B.Cu) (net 9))
 (segment (start 128.73 106.665) (end 127.269 106.665) (width 0.25) (layer F.Cu) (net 9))
 (segment (start 127.254 106.68) (end 126.619 107.315) (width 0.25) (layer B.Cu) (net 9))
 (via (at 127.254 106.68) (size 0.6) (drill 0.4) (layers F.Cu B.Cu) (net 9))
 (segment (start 127.269 106.665) (end 127.254 106.68) (width 0.25) (layer F.Cu) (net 9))
 (segment (start 126.619 107.315) (end 125.99416 107.315) (width 0.25) (layer B.Cu) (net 9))
 (segment (start 127.254 105.41) (end 128.51384 105.41) (width 0.25) (layer B.Cu) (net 10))
 (segment (start 125.99416 105.41) (end 127.254 105.41) (width 0.25) (layer B.Cu) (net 10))
 (segment (start 127.351 106.015) (end 128.73 106.015) (width 0.25) (layer F.Cu) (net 10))
 (segment (start 127.254 105.918) (end 127.351 106.015) (width 0.25) (layer F.Cu) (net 10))
 (segment (start 127.254 105.41) (end 127.254 105.918) (width 0.25) (layer F.Cu) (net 10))
 (via (at 127.254 105.41) (size 0.6) (drill 0.4) (layers F.Cu B.Cu) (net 10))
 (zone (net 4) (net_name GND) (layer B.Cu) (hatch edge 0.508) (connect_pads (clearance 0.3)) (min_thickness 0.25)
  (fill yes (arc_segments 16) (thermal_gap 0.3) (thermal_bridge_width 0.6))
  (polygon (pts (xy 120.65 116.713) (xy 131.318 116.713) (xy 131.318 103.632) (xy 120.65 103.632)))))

